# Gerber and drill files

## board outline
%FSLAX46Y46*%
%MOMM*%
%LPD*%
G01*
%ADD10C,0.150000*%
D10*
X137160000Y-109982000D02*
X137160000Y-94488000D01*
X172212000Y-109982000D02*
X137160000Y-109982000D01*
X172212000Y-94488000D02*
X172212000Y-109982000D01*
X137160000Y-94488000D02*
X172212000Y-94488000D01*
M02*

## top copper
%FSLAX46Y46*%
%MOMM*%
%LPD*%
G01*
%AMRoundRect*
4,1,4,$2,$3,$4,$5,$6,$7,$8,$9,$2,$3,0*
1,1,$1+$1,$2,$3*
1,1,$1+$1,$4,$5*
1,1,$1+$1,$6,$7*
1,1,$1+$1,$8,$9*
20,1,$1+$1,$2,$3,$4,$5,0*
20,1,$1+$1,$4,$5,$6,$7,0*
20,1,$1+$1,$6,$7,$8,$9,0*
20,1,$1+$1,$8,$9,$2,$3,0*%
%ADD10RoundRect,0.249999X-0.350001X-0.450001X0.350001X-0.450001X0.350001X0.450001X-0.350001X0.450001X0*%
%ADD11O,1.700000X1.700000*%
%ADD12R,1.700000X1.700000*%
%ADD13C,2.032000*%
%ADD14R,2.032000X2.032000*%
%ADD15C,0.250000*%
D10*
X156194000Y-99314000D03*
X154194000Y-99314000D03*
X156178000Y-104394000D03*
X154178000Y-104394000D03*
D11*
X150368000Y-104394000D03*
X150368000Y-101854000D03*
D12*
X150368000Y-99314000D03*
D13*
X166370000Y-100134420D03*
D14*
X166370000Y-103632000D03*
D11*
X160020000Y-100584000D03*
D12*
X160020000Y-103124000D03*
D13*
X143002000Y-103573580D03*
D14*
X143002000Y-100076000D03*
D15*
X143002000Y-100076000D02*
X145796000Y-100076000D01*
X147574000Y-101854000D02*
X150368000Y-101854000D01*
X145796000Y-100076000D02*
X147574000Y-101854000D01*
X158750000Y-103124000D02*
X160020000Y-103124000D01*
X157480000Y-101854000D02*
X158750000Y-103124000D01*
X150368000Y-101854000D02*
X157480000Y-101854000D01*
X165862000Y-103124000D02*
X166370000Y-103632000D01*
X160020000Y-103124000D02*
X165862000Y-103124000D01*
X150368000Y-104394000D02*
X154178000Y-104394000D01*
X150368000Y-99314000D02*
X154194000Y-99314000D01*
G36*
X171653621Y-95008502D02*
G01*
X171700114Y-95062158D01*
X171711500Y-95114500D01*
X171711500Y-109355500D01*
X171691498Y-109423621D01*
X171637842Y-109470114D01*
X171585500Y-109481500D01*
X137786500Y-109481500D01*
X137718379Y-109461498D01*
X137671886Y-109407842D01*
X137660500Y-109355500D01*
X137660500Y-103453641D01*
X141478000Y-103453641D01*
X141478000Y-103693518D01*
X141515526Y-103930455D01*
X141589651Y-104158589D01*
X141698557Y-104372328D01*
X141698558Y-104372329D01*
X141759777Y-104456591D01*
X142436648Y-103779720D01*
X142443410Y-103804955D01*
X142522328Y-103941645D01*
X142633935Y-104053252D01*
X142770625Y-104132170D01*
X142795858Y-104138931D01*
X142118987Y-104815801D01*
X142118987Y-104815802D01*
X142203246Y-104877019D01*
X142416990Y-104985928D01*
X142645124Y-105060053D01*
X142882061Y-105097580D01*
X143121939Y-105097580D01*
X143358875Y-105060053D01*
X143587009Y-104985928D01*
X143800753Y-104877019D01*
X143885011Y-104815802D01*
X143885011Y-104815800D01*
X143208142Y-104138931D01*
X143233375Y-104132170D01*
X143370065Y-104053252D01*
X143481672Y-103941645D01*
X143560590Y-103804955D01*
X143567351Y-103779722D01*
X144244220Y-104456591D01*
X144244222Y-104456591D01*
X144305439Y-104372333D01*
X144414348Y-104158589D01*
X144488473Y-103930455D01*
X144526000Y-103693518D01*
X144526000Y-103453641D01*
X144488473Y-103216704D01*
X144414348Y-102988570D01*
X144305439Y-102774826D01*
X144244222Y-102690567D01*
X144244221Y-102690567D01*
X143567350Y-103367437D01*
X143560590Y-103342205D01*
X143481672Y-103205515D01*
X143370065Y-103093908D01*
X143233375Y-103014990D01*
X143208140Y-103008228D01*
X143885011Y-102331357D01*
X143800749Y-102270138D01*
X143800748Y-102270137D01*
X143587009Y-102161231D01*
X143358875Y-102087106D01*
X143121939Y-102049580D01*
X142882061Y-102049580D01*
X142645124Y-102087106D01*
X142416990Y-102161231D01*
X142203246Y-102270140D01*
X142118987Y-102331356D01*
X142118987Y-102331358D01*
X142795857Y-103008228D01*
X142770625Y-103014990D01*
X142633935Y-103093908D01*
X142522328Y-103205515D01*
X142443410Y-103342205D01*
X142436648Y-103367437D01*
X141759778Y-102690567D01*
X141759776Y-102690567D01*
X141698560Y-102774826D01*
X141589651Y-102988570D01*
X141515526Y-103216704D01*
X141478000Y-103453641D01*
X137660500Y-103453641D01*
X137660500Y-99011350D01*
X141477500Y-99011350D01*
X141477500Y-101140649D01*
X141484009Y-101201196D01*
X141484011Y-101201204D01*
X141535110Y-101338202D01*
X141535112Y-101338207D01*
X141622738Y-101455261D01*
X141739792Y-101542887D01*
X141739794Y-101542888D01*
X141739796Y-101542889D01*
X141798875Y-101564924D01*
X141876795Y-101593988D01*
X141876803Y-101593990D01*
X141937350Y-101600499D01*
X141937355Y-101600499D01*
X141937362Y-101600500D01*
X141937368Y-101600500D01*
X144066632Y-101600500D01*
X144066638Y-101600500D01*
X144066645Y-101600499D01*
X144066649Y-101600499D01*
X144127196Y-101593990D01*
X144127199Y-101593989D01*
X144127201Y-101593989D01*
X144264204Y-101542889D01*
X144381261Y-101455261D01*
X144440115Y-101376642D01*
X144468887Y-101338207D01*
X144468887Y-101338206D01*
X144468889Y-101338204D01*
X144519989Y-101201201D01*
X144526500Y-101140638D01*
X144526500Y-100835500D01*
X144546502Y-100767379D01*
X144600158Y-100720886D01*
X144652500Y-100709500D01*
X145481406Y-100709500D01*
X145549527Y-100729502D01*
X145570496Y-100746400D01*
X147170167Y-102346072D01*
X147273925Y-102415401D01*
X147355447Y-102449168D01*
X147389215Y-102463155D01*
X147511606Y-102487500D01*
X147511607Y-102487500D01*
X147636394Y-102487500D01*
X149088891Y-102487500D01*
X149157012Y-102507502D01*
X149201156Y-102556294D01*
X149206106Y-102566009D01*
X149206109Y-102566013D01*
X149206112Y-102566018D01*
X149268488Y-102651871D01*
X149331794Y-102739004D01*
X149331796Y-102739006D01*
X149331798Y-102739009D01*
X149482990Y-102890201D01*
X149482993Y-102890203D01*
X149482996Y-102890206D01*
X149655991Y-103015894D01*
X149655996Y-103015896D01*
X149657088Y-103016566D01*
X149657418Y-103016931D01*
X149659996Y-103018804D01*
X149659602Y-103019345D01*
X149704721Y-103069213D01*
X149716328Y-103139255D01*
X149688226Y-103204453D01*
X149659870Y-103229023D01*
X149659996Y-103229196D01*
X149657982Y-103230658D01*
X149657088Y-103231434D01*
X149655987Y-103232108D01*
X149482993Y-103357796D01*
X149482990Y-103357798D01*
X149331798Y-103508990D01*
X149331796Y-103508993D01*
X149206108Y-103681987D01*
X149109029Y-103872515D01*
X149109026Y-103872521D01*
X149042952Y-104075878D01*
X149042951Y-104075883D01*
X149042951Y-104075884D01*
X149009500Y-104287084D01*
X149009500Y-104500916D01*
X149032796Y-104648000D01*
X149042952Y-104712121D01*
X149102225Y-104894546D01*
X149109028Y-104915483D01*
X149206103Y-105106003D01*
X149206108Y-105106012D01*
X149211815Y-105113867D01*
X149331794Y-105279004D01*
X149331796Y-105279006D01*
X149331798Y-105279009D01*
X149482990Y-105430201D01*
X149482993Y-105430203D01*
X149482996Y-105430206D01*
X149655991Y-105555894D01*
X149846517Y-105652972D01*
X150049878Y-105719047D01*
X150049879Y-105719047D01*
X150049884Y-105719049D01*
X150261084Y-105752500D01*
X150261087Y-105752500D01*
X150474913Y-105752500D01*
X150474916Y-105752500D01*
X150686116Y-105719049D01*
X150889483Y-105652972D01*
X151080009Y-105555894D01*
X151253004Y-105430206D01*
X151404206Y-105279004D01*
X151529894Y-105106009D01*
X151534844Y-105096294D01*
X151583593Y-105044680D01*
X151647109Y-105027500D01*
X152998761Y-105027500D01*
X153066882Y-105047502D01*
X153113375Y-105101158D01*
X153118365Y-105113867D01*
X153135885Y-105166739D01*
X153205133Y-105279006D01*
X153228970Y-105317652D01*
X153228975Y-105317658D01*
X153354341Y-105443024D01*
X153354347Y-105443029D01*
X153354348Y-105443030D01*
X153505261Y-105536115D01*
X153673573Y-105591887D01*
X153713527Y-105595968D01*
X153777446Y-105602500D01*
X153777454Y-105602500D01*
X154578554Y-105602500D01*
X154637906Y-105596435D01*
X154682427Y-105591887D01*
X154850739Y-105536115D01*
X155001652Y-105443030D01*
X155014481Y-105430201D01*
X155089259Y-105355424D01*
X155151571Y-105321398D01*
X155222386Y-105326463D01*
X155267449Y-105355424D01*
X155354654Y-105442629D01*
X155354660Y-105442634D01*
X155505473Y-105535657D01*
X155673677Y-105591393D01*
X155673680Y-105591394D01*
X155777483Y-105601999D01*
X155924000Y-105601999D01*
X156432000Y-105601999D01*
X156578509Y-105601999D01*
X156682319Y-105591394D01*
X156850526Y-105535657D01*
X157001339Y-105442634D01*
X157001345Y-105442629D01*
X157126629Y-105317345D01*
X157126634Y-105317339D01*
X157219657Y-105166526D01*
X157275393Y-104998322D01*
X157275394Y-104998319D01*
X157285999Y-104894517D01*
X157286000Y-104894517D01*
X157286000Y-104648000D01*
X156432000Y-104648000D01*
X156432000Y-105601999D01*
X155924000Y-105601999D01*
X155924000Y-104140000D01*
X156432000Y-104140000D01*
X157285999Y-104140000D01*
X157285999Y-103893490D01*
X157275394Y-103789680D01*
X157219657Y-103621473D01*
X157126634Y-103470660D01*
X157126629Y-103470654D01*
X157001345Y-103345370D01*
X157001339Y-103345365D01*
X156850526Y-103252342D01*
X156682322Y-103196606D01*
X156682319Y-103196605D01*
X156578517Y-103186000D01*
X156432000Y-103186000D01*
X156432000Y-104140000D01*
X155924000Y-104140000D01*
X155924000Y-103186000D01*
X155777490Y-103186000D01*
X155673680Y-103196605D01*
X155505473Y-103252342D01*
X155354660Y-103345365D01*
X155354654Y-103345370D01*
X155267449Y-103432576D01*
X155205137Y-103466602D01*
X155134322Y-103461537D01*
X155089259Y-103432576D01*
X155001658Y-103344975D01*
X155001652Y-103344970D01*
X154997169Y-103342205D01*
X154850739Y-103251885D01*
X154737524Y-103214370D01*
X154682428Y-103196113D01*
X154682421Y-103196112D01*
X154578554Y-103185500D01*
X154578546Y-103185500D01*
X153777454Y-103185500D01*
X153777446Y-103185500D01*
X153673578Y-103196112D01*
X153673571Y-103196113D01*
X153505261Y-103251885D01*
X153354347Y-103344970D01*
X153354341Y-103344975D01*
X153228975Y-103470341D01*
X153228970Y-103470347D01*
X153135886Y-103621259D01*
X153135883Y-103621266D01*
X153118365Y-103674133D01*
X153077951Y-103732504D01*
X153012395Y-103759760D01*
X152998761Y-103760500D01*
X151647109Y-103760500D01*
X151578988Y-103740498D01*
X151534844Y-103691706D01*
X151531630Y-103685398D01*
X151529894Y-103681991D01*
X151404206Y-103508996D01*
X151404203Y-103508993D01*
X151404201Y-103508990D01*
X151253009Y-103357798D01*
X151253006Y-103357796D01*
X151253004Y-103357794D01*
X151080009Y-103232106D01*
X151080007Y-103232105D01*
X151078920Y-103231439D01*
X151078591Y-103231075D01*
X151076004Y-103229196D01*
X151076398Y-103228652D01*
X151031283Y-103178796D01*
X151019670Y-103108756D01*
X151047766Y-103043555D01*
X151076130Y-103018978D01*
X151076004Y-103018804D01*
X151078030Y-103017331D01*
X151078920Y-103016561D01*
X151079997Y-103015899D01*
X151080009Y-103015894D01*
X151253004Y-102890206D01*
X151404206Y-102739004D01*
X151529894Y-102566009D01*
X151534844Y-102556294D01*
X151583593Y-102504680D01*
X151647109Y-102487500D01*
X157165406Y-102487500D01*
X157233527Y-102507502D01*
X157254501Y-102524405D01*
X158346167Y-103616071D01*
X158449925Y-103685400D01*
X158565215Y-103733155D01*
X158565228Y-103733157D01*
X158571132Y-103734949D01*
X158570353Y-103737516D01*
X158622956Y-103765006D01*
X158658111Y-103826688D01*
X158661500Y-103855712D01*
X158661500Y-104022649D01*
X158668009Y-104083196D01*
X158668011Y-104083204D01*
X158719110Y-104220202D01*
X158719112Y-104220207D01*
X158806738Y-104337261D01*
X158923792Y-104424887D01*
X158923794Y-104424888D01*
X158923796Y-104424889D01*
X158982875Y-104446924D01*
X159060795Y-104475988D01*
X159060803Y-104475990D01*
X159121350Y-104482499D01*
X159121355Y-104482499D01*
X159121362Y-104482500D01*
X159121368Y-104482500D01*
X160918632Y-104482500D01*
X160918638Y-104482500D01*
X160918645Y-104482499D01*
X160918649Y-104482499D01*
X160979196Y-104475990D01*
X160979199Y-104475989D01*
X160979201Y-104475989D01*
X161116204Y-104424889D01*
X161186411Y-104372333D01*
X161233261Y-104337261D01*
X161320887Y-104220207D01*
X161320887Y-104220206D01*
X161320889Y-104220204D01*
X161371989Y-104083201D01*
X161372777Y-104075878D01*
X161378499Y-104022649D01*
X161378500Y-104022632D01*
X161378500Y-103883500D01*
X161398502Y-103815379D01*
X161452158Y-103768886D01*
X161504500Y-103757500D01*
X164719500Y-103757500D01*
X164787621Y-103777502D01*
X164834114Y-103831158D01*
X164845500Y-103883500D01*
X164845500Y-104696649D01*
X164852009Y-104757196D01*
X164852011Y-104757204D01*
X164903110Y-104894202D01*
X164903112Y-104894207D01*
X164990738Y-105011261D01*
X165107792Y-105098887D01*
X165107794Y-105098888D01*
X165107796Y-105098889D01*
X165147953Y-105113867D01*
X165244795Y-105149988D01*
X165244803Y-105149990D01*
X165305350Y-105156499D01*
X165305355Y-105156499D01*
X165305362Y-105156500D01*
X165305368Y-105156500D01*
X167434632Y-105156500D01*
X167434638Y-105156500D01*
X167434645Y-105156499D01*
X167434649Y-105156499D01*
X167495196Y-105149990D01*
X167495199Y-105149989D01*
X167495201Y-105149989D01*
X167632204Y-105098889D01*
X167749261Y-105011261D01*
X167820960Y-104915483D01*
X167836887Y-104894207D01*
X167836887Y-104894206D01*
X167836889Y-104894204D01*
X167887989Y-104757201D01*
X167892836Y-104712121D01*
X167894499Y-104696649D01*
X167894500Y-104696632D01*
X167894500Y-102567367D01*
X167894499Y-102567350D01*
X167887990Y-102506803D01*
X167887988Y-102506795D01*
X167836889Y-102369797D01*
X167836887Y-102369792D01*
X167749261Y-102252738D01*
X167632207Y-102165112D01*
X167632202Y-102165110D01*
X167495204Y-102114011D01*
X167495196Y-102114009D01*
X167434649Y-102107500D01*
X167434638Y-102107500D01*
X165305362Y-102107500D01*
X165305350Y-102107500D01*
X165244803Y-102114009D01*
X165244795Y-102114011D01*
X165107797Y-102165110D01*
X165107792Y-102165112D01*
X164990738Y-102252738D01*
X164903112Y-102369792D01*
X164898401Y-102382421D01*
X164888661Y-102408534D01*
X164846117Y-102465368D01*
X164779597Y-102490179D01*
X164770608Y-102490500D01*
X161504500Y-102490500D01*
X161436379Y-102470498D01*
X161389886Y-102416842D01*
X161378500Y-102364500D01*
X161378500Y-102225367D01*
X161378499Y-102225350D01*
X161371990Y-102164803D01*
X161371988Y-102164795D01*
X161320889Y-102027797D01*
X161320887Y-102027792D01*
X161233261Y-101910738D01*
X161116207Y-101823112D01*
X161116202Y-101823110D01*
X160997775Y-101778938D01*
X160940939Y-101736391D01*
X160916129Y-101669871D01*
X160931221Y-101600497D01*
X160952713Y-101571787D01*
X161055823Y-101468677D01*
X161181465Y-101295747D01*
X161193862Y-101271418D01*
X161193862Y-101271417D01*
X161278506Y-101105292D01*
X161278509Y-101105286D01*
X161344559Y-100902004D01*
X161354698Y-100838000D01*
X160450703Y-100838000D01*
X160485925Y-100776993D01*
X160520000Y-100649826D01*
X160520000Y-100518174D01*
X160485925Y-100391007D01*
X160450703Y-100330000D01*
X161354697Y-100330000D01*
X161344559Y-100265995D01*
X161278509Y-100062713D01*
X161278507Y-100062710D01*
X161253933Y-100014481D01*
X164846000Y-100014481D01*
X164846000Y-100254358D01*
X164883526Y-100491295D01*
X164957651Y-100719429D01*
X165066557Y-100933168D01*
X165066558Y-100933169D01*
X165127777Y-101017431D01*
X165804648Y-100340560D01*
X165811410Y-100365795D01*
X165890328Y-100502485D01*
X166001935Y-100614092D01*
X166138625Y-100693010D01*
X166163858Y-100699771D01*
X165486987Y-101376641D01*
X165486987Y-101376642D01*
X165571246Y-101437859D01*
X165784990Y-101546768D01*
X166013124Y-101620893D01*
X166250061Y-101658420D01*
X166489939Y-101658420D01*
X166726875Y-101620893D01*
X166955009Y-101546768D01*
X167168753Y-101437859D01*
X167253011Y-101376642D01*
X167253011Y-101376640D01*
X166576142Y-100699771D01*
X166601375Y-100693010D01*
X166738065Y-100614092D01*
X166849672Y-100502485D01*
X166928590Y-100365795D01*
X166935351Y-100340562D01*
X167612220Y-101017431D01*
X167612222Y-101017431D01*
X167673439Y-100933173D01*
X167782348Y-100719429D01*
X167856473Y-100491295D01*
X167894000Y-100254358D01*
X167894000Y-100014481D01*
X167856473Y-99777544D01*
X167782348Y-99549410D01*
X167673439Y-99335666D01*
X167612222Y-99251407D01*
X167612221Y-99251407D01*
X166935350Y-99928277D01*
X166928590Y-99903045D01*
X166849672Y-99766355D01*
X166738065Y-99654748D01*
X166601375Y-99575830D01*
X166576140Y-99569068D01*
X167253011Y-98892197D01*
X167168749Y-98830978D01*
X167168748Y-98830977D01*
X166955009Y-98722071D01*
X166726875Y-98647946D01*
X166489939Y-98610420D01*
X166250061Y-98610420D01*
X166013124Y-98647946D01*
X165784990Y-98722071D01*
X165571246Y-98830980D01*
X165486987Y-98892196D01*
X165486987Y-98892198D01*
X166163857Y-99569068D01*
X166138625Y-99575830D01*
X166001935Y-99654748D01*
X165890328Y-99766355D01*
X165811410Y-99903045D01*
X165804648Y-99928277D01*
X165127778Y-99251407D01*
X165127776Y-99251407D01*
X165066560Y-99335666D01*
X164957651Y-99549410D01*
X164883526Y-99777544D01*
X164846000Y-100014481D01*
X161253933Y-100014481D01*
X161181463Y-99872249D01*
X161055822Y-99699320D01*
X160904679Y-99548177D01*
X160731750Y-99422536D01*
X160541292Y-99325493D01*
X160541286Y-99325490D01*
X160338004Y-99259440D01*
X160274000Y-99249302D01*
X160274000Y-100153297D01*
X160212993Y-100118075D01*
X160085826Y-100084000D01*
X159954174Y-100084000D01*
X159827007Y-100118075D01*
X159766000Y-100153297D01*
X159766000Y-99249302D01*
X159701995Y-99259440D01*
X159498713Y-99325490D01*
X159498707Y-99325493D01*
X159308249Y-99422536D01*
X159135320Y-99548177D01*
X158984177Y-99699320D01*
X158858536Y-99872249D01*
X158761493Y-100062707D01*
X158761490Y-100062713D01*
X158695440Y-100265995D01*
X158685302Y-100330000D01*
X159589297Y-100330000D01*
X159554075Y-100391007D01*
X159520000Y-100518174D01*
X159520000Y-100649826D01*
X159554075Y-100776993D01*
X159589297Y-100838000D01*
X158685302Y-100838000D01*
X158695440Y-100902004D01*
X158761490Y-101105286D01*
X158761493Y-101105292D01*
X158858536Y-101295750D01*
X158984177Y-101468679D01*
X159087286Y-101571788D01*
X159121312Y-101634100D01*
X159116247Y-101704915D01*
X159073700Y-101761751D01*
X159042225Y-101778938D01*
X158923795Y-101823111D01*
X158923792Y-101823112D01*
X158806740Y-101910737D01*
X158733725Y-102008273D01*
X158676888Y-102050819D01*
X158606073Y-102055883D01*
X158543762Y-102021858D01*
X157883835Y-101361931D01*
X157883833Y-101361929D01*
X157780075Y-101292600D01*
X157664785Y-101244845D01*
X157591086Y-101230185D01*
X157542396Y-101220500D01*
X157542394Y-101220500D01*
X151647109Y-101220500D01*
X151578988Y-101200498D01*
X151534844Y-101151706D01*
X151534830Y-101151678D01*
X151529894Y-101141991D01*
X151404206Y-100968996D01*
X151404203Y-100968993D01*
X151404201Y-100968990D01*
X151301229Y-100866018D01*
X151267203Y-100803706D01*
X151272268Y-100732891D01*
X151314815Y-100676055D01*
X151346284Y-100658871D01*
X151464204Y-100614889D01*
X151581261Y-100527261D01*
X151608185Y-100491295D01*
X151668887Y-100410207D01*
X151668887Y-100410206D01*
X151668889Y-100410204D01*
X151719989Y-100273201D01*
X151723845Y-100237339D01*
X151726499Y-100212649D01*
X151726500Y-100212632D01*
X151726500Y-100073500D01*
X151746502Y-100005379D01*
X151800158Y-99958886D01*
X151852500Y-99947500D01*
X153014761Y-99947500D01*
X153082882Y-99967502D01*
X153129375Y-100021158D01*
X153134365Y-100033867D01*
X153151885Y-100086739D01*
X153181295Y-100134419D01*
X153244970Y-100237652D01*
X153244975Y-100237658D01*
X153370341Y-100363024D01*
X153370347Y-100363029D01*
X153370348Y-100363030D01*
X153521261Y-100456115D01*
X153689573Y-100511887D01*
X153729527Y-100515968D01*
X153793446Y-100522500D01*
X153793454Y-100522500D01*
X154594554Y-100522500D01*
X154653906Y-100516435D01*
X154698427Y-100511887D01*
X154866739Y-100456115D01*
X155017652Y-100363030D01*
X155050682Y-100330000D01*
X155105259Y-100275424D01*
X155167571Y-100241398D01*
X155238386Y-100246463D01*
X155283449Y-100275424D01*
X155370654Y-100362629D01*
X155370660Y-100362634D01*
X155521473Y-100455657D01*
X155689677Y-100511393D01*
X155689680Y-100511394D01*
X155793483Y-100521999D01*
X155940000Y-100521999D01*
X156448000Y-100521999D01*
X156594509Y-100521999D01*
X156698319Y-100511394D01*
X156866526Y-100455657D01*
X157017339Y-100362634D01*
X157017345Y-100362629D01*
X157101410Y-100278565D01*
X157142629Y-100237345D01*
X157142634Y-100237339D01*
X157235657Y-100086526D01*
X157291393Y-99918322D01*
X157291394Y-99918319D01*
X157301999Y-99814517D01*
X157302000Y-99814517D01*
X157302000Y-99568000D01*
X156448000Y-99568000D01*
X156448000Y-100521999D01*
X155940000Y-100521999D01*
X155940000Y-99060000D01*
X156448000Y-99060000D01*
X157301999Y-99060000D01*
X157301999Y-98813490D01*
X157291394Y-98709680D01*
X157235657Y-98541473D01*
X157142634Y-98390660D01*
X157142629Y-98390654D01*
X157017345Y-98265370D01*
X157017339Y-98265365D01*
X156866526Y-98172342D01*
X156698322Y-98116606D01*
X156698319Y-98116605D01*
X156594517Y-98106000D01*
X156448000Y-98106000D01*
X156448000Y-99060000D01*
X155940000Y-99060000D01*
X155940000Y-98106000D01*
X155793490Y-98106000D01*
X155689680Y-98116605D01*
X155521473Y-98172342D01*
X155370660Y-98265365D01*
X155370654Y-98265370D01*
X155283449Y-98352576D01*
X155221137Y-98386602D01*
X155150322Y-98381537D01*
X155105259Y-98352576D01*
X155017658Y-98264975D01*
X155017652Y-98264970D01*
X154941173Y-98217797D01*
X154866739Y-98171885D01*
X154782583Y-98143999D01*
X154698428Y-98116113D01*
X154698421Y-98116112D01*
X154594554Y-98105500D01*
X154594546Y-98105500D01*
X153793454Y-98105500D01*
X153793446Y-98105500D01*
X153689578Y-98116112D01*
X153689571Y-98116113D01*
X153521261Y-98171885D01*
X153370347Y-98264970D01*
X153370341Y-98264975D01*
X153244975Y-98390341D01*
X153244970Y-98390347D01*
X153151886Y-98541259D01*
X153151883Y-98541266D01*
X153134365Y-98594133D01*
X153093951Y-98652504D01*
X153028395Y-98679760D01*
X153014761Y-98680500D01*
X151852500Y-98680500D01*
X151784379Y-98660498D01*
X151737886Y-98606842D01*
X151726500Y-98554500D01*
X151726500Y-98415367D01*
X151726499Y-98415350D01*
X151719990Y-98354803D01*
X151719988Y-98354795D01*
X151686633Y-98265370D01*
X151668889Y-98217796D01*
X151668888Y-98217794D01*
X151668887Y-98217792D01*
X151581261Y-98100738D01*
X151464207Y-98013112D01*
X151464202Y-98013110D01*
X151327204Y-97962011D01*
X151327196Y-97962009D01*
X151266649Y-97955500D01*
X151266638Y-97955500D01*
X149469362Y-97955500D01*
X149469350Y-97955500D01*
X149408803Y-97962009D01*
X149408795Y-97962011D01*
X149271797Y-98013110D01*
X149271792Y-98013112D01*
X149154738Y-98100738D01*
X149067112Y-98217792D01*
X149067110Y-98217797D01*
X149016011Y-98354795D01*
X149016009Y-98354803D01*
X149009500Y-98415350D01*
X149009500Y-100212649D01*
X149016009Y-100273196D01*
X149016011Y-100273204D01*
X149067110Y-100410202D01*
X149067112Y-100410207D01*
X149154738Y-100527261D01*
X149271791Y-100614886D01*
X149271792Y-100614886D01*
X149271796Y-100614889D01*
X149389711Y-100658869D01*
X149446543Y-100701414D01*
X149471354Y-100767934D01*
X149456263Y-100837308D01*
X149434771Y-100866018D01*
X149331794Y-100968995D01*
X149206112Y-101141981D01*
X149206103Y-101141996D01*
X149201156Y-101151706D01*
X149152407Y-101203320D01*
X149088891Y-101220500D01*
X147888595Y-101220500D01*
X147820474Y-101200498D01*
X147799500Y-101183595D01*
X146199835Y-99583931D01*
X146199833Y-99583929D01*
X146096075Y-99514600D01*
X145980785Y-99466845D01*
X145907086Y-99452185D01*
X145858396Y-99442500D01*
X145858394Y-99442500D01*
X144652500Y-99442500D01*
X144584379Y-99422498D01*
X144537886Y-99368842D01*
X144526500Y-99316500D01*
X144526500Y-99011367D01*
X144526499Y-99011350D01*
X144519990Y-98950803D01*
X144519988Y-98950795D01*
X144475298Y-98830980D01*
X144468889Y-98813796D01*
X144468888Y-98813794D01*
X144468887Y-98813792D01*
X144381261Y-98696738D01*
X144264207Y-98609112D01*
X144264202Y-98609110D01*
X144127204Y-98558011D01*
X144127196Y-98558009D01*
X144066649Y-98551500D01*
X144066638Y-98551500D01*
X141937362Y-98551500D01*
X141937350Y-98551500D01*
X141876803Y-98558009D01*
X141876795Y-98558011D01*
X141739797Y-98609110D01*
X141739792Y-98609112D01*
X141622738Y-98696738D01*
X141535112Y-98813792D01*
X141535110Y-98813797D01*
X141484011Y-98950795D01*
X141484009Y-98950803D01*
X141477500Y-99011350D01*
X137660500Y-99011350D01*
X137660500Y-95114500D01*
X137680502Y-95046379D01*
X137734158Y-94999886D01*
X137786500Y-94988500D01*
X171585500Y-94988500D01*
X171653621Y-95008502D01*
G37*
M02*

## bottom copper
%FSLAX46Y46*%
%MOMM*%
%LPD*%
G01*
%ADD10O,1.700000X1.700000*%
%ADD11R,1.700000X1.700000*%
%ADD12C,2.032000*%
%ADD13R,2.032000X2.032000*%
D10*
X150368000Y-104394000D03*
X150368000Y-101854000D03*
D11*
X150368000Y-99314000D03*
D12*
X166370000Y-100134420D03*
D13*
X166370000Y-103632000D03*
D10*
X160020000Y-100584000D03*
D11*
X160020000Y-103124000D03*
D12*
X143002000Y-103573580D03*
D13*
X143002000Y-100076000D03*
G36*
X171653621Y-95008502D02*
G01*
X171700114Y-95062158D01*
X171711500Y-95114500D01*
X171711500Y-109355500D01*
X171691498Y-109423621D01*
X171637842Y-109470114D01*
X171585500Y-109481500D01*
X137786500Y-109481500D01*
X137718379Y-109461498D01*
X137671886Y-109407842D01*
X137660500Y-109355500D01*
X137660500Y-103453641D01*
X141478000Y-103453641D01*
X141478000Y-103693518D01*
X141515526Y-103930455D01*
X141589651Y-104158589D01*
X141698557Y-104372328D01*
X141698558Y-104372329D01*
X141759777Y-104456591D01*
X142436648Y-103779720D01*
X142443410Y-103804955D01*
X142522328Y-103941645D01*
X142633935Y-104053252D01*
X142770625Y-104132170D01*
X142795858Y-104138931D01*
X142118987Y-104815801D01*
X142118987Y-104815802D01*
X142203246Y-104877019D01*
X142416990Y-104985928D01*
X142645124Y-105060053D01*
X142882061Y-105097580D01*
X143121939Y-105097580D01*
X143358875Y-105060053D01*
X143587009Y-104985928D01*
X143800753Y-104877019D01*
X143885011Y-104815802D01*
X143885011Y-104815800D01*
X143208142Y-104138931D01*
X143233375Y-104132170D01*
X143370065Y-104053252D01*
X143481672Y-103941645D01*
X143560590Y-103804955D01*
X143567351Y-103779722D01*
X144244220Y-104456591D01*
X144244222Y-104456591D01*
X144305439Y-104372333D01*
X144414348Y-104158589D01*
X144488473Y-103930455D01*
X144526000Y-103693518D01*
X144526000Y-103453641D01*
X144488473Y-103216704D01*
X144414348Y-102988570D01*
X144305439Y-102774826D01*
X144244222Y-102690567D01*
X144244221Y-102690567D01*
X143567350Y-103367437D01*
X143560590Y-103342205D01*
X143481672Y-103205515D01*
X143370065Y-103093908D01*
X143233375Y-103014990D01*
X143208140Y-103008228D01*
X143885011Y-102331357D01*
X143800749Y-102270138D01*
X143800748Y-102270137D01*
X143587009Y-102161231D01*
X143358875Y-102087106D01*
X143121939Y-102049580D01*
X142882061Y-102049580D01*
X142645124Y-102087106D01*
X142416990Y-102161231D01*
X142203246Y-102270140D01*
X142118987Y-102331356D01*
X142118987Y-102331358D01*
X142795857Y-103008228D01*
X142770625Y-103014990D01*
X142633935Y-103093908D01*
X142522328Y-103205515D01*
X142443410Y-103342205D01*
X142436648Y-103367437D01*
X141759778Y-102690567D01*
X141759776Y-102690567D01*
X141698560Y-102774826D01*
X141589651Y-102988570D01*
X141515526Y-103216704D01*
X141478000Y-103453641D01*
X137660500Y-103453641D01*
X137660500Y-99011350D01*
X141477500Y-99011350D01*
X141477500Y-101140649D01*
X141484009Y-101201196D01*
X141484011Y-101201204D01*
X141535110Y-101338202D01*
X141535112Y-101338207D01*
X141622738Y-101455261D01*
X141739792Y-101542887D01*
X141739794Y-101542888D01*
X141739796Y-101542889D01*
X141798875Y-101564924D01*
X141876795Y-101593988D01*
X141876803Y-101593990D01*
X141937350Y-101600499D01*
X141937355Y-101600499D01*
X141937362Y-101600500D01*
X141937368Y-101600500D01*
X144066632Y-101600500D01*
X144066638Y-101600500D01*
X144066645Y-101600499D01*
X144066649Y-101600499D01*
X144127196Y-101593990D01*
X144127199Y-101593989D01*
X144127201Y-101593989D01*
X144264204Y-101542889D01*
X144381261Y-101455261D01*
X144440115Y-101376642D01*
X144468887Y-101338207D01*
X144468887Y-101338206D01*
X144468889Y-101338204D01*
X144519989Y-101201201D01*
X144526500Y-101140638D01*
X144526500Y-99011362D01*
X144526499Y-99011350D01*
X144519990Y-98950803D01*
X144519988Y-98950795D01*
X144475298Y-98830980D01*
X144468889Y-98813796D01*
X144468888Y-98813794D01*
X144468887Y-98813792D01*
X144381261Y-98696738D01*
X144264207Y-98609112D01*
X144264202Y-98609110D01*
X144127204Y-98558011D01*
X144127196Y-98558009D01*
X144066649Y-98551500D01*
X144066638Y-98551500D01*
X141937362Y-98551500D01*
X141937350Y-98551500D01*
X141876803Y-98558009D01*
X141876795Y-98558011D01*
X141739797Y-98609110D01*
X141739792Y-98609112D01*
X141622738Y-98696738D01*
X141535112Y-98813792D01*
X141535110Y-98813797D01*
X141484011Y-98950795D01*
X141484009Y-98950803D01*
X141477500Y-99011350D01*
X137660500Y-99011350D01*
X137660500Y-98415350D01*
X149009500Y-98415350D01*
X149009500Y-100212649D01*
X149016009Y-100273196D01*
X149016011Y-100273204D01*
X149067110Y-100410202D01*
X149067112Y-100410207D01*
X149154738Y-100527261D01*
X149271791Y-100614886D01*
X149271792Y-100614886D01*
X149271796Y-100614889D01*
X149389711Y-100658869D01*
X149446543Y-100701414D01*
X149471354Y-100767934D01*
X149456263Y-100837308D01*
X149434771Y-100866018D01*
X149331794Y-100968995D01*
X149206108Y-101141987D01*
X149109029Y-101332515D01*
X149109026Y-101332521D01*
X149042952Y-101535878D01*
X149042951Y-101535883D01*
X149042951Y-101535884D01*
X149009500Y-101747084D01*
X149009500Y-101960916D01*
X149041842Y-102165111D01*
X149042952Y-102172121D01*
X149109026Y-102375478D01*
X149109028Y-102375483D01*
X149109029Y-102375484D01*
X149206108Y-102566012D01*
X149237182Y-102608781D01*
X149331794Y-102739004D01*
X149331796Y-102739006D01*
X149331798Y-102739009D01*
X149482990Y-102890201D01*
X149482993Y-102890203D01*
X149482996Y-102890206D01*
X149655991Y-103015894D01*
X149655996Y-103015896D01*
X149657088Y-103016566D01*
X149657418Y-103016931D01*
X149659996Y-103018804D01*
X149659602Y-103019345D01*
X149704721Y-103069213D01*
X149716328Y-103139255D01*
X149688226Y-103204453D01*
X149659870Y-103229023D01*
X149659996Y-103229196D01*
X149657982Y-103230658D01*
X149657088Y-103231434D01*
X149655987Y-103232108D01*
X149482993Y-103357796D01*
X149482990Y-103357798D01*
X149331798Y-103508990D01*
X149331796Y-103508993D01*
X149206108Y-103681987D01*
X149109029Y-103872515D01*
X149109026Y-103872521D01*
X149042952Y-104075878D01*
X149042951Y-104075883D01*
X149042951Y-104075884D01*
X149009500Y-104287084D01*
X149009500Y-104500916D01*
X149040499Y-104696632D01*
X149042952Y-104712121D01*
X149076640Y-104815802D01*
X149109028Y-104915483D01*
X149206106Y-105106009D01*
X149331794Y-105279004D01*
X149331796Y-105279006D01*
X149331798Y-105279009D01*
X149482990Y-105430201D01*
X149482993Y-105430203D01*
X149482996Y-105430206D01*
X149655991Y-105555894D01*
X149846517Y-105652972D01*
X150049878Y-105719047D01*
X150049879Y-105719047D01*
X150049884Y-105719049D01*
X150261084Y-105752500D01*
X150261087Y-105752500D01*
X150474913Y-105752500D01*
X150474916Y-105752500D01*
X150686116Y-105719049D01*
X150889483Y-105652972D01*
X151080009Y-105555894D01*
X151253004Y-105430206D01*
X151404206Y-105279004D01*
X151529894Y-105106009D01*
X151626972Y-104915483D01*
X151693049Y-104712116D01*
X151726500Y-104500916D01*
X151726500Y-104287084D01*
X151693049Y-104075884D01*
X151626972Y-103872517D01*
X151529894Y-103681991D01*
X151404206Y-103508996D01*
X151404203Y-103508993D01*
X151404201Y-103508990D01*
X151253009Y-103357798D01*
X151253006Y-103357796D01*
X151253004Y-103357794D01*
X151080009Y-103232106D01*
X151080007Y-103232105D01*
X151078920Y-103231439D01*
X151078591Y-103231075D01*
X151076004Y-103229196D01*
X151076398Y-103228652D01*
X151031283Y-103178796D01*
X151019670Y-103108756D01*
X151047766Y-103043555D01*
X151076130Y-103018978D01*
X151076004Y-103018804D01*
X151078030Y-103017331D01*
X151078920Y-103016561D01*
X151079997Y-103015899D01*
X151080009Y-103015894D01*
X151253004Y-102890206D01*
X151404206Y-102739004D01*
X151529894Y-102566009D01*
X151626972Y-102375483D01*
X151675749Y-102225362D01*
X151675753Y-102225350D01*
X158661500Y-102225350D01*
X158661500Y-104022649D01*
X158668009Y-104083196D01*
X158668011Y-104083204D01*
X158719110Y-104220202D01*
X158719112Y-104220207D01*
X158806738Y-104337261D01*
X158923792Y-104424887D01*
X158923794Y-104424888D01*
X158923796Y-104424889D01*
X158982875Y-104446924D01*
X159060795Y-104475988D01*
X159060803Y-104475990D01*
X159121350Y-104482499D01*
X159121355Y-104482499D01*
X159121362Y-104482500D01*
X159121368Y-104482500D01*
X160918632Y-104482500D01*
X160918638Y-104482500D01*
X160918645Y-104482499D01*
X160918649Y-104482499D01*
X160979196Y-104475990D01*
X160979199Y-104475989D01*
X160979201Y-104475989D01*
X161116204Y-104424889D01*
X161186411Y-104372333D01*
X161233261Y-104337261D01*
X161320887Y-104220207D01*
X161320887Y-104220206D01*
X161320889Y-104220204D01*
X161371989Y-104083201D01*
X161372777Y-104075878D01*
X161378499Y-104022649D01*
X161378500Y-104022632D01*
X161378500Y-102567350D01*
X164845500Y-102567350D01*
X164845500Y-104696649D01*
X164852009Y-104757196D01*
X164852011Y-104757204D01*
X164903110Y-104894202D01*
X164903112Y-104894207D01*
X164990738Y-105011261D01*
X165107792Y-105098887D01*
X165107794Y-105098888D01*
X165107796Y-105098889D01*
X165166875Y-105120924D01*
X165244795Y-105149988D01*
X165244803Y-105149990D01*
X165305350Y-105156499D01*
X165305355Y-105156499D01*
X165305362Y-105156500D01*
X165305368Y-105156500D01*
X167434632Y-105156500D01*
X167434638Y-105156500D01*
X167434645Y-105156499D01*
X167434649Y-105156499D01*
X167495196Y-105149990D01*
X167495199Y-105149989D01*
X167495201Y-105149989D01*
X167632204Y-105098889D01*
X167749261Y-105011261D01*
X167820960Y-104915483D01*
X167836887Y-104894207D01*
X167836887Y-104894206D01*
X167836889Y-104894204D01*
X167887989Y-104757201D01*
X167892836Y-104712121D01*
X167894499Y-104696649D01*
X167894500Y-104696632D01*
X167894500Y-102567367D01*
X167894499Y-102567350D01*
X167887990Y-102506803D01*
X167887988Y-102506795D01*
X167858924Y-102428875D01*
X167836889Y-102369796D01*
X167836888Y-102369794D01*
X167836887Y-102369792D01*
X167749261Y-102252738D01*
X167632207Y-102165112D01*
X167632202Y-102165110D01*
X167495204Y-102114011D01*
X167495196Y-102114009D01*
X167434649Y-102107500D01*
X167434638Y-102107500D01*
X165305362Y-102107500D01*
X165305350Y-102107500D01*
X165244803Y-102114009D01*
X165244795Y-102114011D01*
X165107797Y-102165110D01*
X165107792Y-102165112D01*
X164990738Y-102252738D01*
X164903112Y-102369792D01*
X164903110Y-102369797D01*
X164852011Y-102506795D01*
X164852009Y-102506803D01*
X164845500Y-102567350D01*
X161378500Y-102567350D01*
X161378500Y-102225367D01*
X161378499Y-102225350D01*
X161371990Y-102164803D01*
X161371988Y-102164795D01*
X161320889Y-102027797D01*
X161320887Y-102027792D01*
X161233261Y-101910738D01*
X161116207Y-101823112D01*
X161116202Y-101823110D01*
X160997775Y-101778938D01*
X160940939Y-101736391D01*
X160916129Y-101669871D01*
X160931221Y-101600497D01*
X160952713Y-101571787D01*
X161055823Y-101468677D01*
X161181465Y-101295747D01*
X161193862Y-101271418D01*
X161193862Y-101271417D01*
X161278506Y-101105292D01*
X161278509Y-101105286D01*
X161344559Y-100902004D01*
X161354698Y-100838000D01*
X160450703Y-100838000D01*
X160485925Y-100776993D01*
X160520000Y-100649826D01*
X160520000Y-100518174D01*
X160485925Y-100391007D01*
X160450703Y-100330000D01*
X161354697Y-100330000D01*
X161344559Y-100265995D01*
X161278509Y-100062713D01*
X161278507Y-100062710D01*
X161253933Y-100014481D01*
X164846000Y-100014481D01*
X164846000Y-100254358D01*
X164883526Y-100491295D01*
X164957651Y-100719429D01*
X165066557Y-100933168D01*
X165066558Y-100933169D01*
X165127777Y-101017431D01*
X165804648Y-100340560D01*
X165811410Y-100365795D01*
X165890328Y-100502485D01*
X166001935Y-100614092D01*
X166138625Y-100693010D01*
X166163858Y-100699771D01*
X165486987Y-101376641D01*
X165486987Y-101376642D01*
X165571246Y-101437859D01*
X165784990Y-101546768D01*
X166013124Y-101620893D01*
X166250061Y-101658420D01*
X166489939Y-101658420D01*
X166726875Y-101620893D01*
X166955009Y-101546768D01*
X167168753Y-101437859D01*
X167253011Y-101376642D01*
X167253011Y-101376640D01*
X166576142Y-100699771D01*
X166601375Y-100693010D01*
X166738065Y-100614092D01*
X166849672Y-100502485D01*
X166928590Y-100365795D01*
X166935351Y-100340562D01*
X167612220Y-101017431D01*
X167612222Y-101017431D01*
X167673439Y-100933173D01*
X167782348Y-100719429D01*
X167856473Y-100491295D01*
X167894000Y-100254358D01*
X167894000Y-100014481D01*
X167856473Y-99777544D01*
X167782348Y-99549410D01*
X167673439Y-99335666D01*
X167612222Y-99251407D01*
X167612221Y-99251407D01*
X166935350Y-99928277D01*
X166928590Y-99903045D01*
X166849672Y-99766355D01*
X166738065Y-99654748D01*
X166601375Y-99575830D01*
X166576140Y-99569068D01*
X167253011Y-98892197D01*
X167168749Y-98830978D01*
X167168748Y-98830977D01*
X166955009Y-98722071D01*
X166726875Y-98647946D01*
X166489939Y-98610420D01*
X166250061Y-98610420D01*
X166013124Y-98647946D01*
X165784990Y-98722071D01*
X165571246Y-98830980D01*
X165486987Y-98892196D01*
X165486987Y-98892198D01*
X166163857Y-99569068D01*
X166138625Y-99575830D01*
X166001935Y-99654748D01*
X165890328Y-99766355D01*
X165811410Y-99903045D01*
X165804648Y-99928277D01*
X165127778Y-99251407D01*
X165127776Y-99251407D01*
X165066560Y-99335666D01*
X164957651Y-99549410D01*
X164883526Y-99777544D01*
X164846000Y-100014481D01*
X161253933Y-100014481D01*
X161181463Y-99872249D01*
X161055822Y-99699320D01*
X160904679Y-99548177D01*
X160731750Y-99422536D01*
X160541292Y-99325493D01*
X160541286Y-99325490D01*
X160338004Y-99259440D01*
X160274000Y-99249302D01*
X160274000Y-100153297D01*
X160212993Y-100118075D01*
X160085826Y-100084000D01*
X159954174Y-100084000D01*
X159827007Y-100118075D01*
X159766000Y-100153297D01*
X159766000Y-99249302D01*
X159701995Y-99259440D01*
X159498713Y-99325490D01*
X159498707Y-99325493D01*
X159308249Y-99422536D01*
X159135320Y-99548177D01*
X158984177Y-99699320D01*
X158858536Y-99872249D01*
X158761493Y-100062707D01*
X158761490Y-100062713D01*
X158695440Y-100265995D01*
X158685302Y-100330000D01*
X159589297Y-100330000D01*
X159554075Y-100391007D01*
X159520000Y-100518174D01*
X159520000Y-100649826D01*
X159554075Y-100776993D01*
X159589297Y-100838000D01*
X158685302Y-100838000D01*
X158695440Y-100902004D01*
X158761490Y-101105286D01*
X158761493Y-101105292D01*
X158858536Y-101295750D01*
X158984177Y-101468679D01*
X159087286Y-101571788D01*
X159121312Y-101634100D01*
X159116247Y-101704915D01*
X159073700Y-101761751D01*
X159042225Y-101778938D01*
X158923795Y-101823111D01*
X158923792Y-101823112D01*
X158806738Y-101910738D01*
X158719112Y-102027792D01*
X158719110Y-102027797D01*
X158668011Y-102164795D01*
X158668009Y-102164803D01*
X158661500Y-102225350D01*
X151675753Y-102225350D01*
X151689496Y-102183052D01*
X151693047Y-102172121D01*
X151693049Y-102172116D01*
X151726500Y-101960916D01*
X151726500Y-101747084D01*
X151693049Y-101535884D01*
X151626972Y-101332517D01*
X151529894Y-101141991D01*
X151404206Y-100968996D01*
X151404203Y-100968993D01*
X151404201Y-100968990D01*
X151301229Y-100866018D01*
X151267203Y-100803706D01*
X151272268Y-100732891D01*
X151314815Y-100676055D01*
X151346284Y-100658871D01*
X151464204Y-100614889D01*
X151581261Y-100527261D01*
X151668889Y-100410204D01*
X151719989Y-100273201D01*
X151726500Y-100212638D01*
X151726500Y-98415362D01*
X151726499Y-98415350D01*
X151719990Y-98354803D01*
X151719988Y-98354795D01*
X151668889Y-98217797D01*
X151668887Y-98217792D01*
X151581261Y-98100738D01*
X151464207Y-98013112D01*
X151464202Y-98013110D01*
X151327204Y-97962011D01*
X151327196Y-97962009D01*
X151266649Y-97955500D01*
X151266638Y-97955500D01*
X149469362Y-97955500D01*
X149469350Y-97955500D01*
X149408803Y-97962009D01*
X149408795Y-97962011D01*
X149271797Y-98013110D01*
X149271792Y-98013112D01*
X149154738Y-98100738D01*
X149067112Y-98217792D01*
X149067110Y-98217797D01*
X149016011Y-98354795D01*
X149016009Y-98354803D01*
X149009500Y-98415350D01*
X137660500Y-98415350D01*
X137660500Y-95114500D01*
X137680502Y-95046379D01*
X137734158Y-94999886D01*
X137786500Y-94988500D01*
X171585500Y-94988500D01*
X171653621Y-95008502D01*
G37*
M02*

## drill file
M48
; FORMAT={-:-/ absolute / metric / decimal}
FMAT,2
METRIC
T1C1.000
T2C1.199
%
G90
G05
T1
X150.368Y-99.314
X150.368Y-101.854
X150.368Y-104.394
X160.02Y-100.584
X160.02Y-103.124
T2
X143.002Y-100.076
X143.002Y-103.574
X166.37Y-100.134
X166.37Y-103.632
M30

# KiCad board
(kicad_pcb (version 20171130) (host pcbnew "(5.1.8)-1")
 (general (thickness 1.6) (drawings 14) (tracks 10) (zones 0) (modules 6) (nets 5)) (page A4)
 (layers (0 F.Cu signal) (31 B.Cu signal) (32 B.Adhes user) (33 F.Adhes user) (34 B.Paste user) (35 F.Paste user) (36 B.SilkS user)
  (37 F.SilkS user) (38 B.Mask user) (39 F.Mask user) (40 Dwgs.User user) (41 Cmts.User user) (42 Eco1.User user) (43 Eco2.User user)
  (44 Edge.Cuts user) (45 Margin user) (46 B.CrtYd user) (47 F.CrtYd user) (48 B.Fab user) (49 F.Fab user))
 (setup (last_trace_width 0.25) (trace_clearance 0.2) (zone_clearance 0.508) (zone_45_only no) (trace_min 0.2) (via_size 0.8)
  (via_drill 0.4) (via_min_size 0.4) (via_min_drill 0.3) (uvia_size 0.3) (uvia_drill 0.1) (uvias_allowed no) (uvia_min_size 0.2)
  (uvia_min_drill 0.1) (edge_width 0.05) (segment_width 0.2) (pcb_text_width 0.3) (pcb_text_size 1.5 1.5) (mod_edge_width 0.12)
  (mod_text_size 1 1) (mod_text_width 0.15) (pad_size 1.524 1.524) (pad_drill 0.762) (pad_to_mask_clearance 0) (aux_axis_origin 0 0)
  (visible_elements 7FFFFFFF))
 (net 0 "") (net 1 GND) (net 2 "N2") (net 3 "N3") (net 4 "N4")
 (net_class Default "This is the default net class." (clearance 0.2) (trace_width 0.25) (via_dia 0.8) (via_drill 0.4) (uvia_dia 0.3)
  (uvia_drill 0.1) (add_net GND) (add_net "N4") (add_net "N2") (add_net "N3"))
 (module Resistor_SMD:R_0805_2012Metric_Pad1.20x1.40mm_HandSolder (layer F.Cu) (at 155.194 99.314)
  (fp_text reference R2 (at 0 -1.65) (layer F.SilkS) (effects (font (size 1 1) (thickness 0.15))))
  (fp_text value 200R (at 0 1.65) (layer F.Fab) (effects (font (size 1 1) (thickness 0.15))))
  (pad 2 smd roundrect (at 1 0) (size 1.2 1.4) (layers F.Cu F.Paste F.Mask) (roundrect_rratio 0.2083325) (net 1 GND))
  (pad 1 smd roundrect (at -1 0) (size 1.2 1.4) (layers F.Cu F.Paste F.Mask) (roundrect_rratio 0.2083325) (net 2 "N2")))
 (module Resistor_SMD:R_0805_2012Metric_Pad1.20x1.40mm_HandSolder (layer F.Cu) (at 155.178 104.394)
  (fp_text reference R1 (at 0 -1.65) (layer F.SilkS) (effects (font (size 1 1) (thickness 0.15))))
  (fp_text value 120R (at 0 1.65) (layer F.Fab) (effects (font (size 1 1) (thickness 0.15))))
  (pad 2 smd roundrect (at 1 0) (size 1.2 1.4) (layers F.Cu F.Paste F.Mask) (roundrect_rratio 0.2083325) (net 1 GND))
  (pad 1 smd roundrect (at -1 0) (size 1.2 1.4) (layers F.Cu F.Paste F.Mask) (roundrect_rratio 0.2083325) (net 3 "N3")))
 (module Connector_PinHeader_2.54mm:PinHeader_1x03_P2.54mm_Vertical (layer F.Cu) (at 150.368 99.314)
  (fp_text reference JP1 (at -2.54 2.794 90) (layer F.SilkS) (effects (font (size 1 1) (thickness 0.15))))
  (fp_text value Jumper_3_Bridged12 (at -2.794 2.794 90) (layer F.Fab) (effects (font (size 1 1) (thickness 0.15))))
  (pad 3 thru_hole oval (at 0 5.08) (size 1.7 1.7) (drill 1) (layers *.Cu *.Mask) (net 3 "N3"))
  (pad 2 thru_hole oval (at 0 2.54) (size 1.7 1.7) (drill 1) (layers *.Cu *.Mask) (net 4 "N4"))
  (pad 1 thru_hole rect (at 0 0) (size 1.7 1.7) (drill 1) (layers *.Cu *.Mask) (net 2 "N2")))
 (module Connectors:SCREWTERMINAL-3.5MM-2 (layer F.Cu) (at 166.37 103.632 90)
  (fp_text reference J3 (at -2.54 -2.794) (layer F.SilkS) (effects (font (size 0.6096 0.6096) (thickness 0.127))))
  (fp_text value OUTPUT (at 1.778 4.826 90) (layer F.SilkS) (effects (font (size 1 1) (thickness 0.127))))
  (pad 2 thru_hole circle (at 3.49758 0 90) (size 2.032 2.032) (drill 1.19888) (layers *.Cu *.Mask) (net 1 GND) (solder_mask_margin 0.1016))
  (pad 1 thru_hole rect (at 0 0 90) (size 2.032 2.032) (drill 1.19888) (layers *.Cu *.Mask) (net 4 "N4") (solder_mask_margin 0.1016)))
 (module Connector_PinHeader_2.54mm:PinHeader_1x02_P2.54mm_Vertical (layer F.Cu) (at 160.02 103.124 180)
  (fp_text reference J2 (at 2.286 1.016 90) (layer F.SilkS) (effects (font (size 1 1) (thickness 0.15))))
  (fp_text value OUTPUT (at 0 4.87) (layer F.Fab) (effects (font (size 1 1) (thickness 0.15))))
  (pad 2 thru_hole oval (at 0 2.54 180) (size 1.7 1.7) (drill 1) (layers *.Cu *.Mask) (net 1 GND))
  (pad 1 thru_hole rect (at 0 0 180) (size 1.7 1.7) (drill 1) (layers *.Cu *.Mask) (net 4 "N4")))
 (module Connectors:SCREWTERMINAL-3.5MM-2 (layer F.Cu) (at 143.002 100.076 270)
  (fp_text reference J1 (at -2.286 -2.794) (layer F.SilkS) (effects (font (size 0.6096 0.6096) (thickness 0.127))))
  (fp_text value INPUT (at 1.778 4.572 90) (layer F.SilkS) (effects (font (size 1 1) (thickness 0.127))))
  (pad 2 thru_hole circle (at 3.49758 0 270) (size 2.032 2.032) (drill 1.19888) (layers *.Cu *.Mask) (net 1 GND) (solder_mask_margin 0.1016))
  (pad 1 thru_hole rect (at 0 0 270) (size 2.032 2.032) (drill 1.19888) (layers *.Cu *.Mask) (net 4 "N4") (solder_mask_margin 0.1016)))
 (gr_line (start 137.16 109.982) (end 137.16 94.488) (layer Edge.Cuts) (width 0.15))
 (gr_line (start 172.212 109.982) (end 137.16 109.982) (layer Edge.Cuts) (width 0.15))
 (gr_line (start 172.212 94.488) (end 172.212 109.982) (layer Edge.Cuts) (width 0.15))
 (gr_line (start 137.16 94.488) (end 172.212 94.488) (layer Edge.Cuts) (width 0.15))
 (segment (start 143.002 100.076) (end 145.796 100.076) (width 0.25) (layer F.Cu) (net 4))
 (segment (start 147.574 101.854) (end 150.368 101.854) (width 0.25) (layer F.Cu) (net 4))
 (segment (start 145.796 100.076) (end 147.574 101.854) (width 0.25) (layer F.Cu) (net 4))
 (segment (start 158.75 103.124) (end 160.02 103.124) (width 0.25) (layer F.Cu) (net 4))
 (segment (start 157.48 101.854) (end 158.75 103.124) (width 0.25) (layer F.Cu) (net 4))
 (segment (start 150.368 101.854) (end 157.48 101.854) (width 0.25) (layer F.Cu) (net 4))
 (segment (start 165.862 103.124) (end 166.37 103.632) (width 0.25) (layer F.Cu) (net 4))
 (segment (start 160.02 103.124) (end 165.862 103.124) (width 0.25) (layer F.Cu) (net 4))
 (segment (start 150.368 104.394) (end 154.178 104.394) (width 0.25) (layer F.Cu) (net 3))
 (segment (start 150.368 99.314) (end 154.194 99.314) (width 0.25) (layer F.Cu) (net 2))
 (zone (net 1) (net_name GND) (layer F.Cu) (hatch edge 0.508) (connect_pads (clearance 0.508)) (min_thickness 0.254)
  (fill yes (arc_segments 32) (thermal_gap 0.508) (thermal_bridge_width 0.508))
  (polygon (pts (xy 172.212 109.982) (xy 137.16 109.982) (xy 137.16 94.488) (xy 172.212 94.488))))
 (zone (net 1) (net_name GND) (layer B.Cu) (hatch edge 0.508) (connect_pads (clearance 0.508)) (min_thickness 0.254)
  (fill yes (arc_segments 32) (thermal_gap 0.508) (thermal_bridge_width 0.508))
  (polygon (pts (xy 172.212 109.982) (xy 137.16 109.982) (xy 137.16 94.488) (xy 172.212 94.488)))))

